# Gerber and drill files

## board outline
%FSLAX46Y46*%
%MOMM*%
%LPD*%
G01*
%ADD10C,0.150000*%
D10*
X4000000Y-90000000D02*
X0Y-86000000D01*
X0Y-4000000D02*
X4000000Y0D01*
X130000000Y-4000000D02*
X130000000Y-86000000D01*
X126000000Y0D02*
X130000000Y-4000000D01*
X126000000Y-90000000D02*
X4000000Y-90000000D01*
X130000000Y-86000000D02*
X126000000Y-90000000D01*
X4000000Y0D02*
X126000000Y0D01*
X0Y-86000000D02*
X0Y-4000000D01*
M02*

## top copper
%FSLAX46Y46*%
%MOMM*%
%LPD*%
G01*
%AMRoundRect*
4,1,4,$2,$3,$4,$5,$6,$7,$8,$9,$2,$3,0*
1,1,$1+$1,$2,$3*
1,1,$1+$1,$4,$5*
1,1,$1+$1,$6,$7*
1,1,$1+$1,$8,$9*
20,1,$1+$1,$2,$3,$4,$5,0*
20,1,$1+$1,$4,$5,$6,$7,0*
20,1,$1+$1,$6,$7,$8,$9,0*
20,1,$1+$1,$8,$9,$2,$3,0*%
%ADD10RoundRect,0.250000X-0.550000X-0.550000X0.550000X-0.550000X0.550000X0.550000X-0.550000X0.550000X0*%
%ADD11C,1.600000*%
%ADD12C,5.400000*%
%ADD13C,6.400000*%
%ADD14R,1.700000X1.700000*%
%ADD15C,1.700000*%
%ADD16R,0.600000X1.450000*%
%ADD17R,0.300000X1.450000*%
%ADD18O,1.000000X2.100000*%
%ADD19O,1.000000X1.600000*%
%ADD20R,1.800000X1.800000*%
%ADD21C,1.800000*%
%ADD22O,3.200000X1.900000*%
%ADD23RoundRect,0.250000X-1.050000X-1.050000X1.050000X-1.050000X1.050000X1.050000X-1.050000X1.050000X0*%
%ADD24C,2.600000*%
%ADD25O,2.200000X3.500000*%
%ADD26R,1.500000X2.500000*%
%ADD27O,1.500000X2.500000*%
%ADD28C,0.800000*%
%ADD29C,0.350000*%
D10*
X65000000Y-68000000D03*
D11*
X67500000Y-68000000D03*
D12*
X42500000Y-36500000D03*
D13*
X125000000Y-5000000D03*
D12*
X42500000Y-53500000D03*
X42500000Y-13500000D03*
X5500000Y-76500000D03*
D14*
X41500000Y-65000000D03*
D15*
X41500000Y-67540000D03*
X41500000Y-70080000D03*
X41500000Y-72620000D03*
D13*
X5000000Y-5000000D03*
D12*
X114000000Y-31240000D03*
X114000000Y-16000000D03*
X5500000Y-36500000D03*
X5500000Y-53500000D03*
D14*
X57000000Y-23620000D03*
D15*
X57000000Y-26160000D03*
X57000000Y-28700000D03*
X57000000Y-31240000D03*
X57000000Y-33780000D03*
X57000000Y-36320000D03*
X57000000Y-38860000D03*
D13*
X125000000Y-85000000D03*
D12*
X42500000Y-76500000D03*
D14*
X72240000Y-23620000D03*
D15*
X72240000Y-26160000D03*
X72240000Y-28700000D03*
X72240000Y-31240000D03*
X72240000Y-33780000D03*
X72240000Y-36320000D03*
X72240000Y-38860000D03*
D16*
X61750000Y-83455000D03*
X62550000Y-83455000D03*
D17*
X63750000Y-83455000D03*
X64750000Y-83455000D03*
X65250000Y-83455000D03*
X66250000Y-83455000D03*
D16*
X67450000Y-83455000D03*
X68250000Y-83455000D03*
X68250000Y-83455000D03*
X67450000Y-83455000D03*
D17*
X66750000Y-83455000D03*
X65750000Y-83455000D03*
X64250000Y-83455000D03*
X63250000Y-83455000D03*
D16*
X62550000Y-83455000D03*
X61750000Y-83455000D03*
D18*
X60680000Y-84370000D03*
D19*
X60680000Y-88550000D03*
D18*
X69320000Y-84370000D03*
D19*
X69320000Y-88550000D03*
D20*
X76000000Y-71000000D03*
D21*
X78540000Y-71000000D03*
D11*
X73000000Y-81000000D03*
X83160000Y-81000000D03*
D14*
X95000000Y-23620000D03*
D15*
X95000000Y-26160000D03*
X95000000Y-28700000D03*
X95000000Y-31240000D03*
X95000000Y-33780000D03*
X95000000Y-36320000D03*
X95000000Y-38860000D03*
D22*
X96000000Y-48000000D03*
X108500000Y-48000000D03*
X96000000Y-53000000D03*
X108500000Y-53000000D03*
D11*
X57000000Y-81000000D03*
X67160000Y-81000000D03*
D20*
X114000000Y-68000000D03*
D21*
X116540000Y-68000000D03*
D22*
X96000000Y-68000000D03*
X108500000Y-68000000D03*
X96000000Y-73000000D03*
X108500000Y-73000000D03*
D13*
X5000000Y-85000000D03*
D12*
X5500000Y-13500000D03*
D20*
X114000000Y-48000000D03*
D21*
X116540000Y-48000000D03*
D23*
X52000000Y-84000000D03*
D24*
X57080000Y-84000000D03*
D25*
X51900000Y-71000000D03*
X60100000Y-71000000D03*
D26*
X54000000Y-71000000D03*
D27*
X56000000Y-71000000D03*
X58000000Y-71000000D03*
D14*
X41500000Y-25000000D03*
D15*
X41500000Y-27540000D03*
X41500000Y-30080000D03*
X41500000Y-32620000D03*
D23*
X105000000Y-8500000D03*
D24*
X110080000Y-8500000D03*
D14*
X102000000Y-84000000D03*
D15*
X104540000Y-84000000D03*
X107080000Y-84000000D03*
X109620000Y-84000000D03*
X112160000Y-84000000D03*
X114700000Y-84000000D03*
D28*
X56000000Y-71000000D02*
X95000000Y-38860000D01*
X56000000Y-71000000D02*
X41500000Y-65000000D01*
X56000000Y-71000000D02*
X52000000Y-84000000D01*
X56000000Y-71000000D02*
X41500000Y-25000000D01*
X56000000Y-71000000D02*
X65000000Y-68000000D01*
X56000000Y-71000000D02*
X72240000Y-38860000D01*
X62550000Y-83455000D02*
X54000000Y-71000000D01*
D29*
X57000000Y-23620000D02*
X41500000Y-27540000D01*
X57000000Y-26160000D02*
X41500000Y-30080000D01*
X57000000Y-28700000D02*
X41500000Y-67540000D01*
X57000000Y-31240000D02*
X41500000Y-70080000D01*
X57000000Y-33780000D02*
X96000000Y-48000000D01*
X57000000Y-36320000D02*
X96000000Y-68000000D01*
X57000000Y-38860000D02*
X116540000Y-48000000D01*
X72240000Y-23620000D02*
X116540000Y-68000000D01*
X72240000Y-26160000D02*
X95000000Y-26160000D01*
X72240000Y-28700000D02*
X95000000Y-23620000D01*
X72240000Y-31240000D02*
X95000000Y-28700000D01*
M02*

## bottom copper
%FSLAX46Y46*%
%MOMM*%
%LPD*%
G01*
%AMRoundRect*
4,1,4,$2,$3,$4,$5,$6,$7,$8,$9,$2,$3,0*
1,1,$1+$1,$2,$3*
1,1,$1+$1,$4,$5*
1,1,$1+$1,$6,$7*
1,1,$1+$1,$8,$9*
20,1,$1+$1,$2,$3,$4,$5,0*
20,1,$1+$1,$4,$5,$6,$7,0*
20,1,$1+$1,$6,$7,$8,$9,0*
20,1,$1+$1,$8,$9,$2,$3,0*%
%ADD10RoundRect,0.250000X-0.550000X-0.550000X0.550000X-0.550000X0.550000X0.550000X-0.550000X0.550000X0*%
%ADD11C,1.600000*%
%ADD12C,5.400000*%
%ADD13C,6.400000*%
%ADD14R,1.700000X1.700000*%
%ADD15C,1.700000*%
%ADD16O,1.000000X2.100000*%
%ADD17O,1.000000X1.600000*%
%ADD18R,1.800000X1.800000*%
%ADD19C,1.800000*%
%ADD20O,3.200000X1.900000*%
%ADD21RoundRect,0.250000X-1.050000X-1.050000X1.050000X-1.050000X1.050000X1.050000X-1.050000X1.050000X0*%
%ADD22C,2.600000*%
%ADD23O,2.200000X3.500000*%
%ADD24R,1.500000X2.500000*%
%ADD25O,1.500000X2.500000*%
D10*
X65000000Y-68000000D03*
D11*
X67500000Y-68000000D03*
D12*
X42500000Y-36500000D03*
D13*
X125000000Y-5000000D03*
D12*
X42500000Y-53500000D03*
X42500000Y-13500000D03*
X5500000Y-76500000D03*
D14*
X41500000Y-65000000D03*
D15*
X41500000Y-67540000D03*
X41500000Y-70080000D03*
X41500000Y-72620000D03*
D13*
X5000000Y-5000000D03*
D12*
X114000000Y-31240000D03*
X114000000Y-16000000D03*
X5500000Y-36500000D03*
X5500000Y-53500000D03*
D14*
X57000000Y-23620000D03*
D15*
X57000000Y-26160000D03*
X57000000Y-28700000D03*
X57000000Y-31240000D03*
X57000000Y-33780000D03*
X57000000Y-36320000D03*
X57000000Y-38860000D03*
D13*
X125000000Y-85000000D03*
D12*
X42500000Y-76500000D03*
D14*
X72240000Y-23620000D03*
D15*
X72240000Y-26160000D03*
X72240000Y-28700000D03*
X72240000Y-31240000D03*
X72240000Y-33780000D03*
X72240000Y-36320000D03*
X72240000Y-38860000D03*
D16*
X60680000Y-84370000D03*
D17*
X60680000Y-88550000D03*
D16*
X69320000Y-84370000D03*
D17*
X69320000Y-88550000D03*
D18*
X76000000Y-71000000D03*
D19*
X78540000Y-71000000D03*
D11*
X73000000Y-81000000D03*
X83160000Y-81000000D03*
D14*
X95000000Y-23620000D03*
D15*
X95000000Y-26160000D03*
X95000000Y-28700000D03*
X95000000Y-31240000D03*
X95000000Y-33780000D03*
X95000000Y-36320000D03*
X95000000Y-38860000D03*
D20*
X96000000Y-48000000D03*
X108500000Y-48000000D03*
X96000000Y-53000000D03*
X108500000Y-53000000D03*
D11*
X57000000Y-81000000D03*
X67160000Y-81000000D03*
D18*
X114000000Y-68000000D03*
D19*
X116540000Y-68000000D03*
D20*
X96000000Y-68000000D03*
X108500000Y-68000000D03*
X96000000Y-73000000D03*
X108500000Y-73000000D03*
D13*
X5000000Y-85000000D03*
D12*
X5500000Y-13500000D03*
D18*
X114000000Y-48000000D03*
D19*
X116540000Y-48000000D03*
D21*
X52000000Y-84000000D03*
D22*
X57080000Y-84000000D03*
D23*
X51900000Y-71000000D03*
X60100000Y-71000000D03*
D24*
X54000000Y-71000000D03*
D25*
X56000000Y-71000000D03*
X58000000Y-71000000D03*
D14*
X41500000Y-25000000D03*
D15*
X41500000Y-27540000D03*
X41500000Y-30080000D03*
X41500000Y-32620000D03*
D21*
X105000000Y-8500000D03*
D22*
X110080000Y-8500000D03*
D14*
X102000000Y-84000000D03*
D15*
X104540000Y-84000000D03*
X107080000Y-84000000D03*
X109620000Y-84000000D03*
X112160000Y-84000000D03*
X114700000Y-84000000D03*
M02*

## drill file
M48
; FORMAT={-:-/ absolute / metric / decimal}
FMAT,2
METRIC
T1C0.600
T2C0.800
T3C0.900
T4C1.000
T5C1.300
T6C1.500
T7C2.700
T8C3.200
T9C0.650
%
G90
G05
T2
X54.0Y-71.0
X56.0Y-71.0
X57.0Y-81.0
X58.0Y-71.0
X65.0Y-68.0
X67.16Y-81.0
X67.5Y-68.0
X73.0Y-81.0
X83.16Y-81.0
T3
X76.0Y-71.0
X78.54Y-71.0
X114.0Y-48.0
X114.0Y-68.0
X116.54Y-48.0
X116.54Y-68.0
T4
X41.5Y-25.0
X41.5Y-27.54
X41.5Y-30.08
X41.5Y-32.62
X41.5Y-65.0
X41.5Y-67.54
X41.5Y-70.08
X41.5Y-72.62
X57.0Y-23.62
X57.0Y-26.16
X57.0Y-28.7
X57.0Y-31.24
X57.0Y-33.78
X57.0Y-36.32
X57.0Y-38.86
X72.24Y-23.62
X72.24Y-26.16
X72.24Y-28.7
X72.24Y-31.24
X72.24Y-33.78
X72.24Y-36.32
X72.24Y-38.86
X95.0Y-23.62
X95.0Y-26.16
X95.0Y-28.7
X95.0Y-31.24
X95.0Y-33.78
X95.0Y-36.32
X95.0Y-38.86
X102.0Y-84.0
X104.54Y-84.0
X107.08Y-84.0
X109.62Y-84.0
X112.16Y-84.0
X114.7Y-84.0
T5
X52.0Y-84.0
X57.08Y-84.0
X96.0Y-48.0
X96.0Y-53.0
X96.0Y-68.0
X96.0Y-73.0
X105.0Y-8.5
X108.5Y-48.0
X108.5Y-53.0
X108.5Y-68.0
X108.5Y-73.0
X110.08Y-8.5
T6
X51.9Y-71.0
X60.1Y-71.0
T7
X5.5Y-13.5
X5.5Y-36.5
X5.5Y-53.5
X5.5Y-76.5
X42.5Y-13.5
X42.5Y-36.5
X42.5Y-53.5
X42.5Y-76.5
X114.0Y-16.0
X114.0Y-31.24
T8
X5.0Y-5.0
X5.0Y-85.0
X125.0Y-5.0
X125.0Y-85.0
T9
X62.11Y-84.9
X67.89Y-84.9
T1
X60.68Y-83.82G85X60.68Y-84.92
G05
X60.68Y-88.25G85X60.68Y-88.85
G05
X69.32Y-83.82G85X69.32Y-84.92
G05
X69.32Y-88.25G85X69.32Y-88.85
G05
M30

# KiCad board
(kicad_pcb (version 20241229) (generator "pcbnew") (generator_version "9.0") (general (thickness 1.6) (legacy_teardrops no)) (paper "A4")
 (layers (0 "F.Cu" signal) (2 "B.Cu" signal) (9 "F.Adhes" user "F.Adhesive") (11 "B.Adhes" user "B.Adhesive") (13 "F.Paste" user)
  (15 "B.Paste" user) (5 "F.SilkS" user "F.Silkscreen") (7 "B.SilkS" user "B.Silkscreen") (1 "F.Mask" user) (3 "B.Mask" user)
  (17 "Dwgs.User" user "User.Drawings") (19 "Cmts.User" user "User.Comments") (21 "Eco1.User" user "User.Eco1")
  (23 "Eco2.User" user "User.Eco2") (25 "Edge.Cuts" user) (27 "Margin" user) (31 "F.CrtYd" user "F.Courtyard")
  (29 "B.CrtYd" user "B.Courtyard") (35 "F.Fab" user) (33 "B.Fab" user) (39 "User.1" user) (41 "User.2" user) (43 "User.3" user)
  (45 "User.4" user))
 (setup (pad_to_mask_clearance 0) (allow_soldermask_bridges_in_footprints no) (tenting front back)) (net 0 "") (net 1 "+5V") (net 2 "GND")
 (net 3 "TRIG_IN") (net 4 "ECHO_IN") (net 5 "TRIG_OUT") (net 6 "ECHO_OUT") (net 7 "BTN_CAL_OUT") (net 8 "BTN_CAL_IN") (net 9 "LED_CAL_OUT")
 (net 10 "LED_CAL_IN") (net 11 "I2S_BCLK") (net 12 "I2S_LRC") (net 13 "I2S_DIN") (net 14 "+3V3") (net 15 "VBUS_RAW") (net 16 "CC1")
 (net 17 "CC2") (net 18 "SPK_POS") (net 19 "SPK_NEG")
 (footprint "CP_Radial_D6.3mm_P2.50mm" (layer "F.Cu") (at 65 68)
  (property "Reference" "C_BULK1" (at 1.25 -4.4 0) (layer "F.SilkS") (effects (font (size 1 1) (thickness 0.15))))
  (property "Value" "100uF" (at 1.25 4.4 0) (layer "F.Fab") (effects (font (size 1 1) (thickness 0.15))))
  (pad "1" thru_hole roundrect (at 0 0) (size 1.6 1.6) (drill 0.8) (layers "*.Cu" "*.Mask") (remove_unused_layers no)
   (roundrect_rratio 0.15625) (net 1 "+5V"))
  (pad "2" thru_hole circle (at 2.5 0) (size 1.6 1.6) (drill 0.8) (layers "*.Cu" "*.Mask") (remove_unused_layers no) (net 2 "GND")))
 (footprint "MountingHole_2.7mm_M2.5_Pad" (layer "F.Cu") (at 42.5 36.5)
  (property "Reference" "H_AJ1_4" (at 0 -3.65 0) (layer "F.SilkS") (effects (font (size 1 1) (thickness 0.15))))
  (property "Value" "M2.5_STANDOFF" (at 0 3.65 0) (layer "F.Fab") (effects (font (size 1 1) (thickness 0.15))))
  (pad "1" thru_hole circle (at 0 0) (size 5.4 5.4) (drill 2.7) (layers "*.Cu" "*.Mask") (remove_unused_layers no) (zone_connect 2)))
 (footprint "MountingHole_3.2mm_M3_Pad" (layer "F.Cu") (at 125 5)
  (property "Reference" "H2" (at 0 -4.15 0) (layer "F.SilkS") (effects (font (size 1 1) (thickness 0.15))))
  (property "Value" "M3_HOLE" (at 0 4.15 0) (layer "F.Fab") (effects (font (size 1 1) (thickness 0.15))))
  (pad "1" thru_hole circle (at 0 0) (size 6.4 6.4) (drill 3.2) (layers "*.Cu" "*.Mask") (remove_unused_layers no) (zone_connect 2)))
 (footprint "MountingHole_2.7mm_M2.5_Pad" (layer "F.Cu") (at 42.5 53.5)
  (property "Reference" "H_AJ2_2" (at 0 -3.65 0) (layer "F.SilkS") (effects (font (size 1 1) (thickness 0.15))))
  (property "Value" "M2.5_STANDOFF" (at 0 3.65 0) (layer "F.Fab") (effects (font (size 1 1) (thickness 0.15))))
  (pad "1" thru_hole circle (at 0 0) (size 5.4 5.4) (drill 2.7) (layers "*.Cu" "*.Mask") (remove_unused_layers no) (zone_connect 2)))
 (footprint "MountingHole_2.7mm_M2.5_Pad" (layer "F.Cu") (at 42.5 13.5)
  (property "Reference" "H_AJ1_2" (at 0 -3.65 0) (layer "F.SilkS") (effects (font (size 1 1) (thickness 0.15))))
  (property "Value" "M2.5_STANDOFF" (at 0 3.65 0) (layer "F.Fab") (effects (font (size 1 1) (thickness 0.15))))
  (pad "1" thru_hole circle (at 0 0) (size 5.4 5.4) (drill 2.7) (layers "*.Cu" "*.Mask") (remove_unused_layers no) (zone_connect 2)))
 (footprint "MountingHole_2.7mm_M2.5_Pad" (layer "F.Cu") (at 5.5 76.5)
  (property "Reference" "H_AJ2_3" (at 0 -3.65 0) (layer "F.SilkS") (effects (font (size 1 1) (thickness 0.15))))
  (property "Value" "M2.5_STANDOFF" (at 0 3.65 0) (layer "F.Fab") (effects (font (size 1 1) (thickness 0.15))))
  (pad "1" thru_hole circle (at 0 0) (size 5.4 5.4) (drill 2.7) (layers "*.Cu" "*.Mask") (remove_unused_layers no) (zone_connect 2)))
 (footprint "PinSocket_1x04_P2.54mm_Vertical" (layer "F.Cu") (at 41.5 65)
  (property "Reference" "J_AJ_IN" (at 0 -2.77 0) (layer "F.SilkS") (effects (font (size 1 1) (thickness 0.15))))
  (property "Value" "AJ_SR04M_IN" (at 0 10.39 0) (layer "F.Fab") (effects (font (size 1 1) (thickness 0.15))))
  (pad "1" thru_hole rect (at 0 0) (size 1.7 1.7) (drill 1) (layers "*.Cu" "*.Mask") (remove_unused_layers no) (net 1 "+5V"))
  (pad "2" thru_hole circle (at 0 2.54) (size 1.7 1.7) (drill 1) (layers "*.Cu" "*.Mask") (remove_unused_layers no) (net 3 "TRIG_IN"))
  (pad "3" thru_hole circle (at 0 5.08) (size 1.7 1.7) (drill 1) (layers "*.Cu" "*.Mask") (remove_unused_layers no) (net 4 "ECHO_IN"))
  (pad "4" thru_hole circle (at 0 7.62) (size 1.7 1.7) (drill 1) (layers "*.Cu" "*.Mask") (remove_unused_layers no) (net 2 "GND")))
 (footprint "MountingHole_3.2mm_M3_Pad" (layer "F.Cu") (at 5 5)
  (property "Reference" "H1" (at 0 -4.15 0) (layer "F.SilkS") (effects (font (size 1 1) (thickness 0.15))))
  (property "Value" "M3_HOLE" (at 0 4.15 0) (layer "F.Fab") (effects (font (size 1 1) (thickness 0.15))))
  (pad "1" thru_hole circle (at 0 0) (size 6.4 6.4) (drill 3.2) (layers "*.Cu" "*.Mask") (remove_unused_layers no) (zone_connect 2)))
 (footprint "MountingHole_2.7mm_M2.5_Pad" (layer "F.Cu") (at 114 31.24)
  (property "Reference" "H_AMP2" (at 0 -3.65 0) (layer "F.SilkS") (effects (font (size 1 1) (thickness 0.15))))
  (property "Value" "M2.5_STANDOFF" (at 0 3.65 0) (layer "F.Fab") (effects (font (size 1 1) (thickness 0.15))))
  (pad "1" thru_hole circle (at 0 0) (size 5.4 5.4) (drill 2.7) (layers "*.Cu" "*.Mask") (remove_unused_layers no) (zone_connect 2)))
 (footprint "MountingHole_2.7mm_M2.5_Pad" (layer "F.Cu") (at 114 16)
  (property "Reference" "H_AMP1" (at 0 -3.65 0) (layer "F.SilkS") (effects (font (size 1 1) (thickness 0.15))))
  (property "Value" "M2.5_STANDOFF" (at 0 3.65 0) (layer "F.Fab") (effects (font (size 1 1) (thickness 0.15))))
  (pad "1" thru_hole circle (at 0 0) (size 5.4 5.4) (drill 2.7) (layers "*.Cu" "*.Mask") (remove_unused_layers no) (zone_connect 2)))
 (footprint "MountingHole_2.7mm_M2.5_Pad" (layer "F.Cu") (at 5.5 36.5)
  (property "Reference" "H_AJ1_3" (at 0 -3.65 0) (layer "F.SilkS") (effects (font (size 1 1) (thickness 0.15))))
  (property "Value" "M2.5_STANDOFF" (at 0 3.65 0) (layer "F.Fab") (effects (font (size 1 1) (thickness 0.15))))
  (pad "1" thru_hole circle (at 0 0) (size 5.4 5.4) (drill 2.7) (layers "*.Cu" "*.Mask") (remove_unused_layers no) (zone_connect 2)))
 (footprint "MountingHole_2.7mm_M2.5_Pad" (layer "F.Cu") (at 5.5 53.5)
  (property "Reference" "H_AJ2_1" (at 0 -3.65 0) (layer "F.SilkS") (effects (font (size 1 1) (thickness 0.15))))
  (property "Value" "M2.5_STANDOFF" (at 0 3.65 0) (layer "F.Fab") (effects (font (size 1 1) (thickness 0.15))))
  (pad "1" thru_hole circle (at 0 0) (size 5.4 5.4) (drill 2.7) (layers "*.Cu" "*.Mask") (remove_unused_layers no) (zone_connect 2)))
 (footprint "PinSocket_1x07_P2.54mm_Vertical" (layer "F.Cu") (at 57 23.62)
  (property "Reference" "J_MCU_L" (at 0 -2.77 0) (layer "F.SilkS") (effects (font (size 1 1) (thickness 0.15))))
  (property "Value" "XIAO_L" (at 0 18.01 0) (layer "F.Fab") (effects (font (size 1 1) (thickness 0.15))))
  (pad "1" thru_hole rect (at 0 0) (size 1.7 1.7) (drill 1) (layers "*.Cu" "*.Mask") (remove_unused_layers no) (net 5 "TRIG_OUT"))
  (pad "2" thru_hole circle (at 0 2.54) (size 1.7 1.7) (drill 1) (layers "*.Cu" "*.Mask") (remove_unused_layers no) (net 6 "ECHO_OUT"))
  (pad "3" thru_hole circle (at 0 5.08) (size 1.7 1.7) (drill 1) (layers "*.Cu" "*.Mask") (remove_unused_layers no) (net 3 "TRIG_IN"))
  (pad "4" thru_hole circle (at 0 7.62) (size 1.7 1.7) (drill 1) (layers "*.Cu" "*.Mask") (remove_unused_layers no) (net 4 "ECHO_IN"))
  (pad "5" thru_hole circle (at 0 10.16) (size 1.7 1.7) (drill 1) (layers "*.Cu" "*.Mask") (remove_unused_layers no) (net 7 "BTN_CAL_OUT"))
  (pad "6" thru_hole circle (at 0 12.7) (size 1.7 1.7) (drill 1) (layers "*.Cu" "*.Mask") (remove_unused_layers no) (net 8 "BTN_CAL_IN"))
  (pad "7" thru_hole circle (at 0 15.24) (size 1.7 1.7) (drill 1) (layers "*.Cu" "*.Mask") (remove_unused_layers no) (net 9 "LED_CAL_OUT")))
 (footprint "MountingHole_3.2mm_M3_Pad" (layer "F.Cu") (at 125 85)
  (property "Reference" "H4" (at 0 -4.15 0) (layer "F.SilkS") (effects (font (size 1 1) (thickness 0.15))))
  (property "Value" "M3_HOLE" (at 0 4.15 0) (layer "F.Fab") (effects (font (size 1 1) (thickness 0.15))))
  (pad "1" thru_hole circle (at 0 0) (size 6.4 6.4) (drill 3.2) (layers "*.Cu" "*.Mask") (remove_unused_layers no) (zone_connect 2)))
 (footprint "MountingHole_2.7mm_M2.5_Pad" (layer "F.Cu") (at 42.5 76.5)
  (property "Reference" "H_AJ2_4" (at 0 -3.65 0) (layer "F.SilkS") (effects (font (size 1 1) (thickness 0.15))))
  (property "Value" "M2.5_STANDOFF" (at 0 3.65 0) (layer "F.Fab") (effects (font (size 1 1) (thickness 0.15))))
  (pad "1" thru_hole circle (at 0 0) (size 5.4 5.4) (drill 2.7) (layers "*.Cu" "*.Mask") (remove_unused_layers no) (zone_connect 2)))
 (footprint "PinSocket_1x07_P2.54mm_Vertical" (layer "F.Cu") (at 72.24 23.62)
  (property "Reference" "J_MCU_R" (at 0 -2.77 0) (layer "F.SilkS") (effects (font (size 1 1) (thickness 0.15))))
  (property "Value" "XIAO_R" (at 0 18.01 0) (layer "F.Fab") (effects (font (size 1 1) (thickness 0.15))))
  (pad "1" thru_hole rect (at 0 0) (size 1.7 1.7) (drill 1) (layers "*.Cu" "*.Mask") (remove_unused_layers no) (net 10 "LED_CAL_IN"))
  (pad "2" thru_hole circle (at 0 2.54) (size 1.7 1.7) (drill 1) (layers "*.Cu" "*.Mask") (remove_unused_layers no) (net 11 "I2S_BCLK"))
  (pad "3" thru_hole circle (at 0 5.08) (size 1.7 1.7) (drill 1) (layers "*.Cu" "*.Mask") (remove_unused_layers no) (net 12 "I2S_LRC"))
  (pad "4" thru_hole circle (at 0 7.62) (size 1.7 1.7) (drill 1) (layers "*.Cu" "*.Mask") (remove_unused_layers no) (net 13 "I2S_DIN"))
  (pad "5" thru_hole circle (at 0 10.16) (size 1.7 1.7) (drill 1) (layers "*.Cu" "*.Mask") (remove_unused_layers no) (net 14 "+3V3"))
  (pad "6" thru_hole circle (at 0 12.7) (size 1.7 1.7) (drill 1) (layers "*.Cu" "*.Mask") (remove_unused_layers no) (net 2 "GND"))
  (pad "7" thru_hole circle (at 0 15.24) (size 1.7 1.7) (drill 1) (layers "*.Cu" "*.Mask") (remove_unused_layers no) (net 1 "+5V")))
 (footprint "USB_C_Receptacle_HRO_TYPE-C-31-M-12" (layer "F.Cu") (at 65 87.5)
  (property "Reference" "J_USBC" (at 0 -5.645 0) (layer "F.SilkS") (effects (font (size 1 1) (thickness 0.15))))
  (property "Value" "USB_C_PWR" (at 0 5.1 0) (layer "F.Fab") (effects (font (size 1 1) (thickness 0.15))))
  (pad "" np_thru_hole circle (at -2.89 -2.6) (size 0.65 0.65) (drill 0.65) (layers "*.Cu" "*.Mask"))
  (pad "" np_thru_hole circle (at 2.89 -2.6) (size 0.65 0.65) (drill 0.65) (layers "*.Cu" "*.Mask"))
  (pad "A1" smd rect (at -3.25 -4.045) (size 0.6 1.45) (layers "F.Cu" "F.Mask" "F.Paste") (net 2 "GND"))
  (pad "A4" smd rect (at -2.45 -4.045) (size 0.6 1.45) (layers "F.Cu" "F.Mask" "F.Paste") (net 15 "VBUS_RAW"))
  (pad "A5" smd rect (at -1.25 -4.045) (size 0.3 1.45) (layers "F.Cu" "F.Mask" "F.Paste") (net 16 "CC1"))
  (pad "A6" smd rect (at -0.25 -4.045) (size 0.3 1.45) (layers "F.Cu" "F.Mask" "F.Paste"))
  (pad "A7" smd rect (at 0.25 -4.045) (size 0.3 1.45) (layers "F.Cu" "F.Mask" "F.Paste"))
  (pad "A8" smd rect (at 1.25 -4.045) (size 0.3 1.45) (layers "F.Cu" "F.Mask" "F.Paste"))
  (pad "A9" smd rect (at 2.45 -4.045) (size 0.6 1.45) (layers "F.Cu" "F.Mask" "F.Paste") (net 15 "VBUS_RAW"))
  (pad "A12" smd rect (at 3.25 -4.045) (size 0.6 1.45) (layers "F.Cu" "F.Mask" "F.Paste") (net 2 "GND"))
  (pad "B1" smd rect (at 3.25 -4.045) (size 0.6 1.45) (layers "F.Cu" "F.Mask" "F.Paste") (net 2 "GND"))
  (pad "B4" smd rect (at 2.45 -4.045) (size 0.6 1.45) (layers "F.Cu" "F.Mask" "F.Paste") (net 15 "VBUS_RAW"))
  (pad "B5" smd rect (at 1.75 -4.045) (size 0.3 1.45) (layers "F.Cu" "F.Mask" "F.Paste") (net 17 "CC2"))
  (pad "B6" smd rect (at 0.75 -4.045) (size 0.3 1.45) (layers "F.Cu" "F.Mask" "F.Paste"))
  (pad "B7" smd rect (at -0.75 -4.045) (size 0.3 1.45) (layers "F.Cu" "F.Mask" "F.Paste"))
  (pad "B8" smd rect (at -1.75 -4.045) (size 0.3 1.45) (layers "F.Cu" "F.Mask" "F.Paste"))
  (pad "B9" smd rect (at -2.45 -4.045) (size 0.6 1.45) (layers "F.Cu" "F.Mask" "F.Paste") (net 15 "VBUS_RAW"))
  (pad "B12" smd rect (at -3.25 -4.045) (size 0.6 1.45) (layers "F.Cu" "F.Mask" "F.Paste") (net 2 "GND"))
  (pad "S1" thru_hole oval (at -4.32 -3.13) (size 1 2.1) (drill oval 0.6 1.7) (layers "*.Cu" "*.Mask") (remove_unused_layers no)
   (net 2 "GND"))
  (pad "S1" thru_hole oval (at -4.32 1.05) (size 1 1.6) (drill oval 0.6 1.2) (layers "*.Cu" "*.Mask") (remove_unused_layers no)
   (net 2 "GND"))
  (pad "S1" thru_hole oval (at 4.32 -3.13) (size 1 2.1) (drill oval 0.6 1.7) (layers "*.Cu" "*.Mask") (remove_unused_layers no)
   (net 2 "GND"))
  (pad "S1" thru_hole oval (at 4.32 1.05) (size 1 1.6) (drill oval 0.6 1.2) (layers "*.Cu" "*.Mask") (remove_unused_layers no) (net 2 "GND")))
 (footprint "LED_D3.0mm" (layer "F.Cu") (at 76 71)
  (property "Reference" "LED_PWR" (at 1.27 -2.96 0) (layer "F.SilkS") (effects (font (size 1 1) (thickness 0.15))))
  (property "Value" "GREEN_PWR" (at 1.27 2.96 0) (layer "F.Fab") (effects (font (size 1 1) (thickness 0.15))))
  (pad "1" thru_hole rect (at 0 0) (size 1.8 1.8) (drill 0.9) (layers "*.Cu" "*.Mask") (remove_unused_layers no) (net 2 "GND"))
  (pad "2" thru_hole circle (at 2.54 0) (size 1.8 1.8) (drill 0.9) (layers "*.Cu" "*.Mask") (remove_unused_layers no) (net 1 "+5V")))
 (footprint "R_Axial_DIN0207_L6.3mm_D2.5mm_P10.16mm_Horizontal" (layer "F.Cu") (at 73 81)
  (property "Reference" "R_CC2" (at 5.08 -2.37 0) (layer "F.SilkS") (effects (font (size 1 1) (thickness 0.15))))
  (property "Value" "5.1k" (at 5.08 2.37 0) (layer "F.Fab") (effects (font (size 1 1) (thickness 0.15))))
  (pad "1" thru_hole circle (at 0 0) (size 1.6 1.6) (drill 0.8) (layers "*.Cu" "*.Mask") (remove_unused_layers no) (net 17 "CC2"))
  (pad "2" thru_hole circle (at 10.16 0) (size 1.6 1.6) (drill 0.8) (layers "*.Cu" "*.Mask") (remove_unused_layers no) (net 2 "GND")))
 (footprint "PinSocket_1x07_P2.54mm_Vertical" (layer "F.Cu") (at 95 23.62)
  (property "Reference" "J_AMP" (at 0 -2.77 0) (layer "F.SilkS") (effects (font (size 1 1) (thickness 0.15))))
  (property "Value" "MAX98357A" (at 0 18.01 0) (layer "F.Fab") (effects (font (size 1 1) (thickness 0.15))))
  (pad "1" thru_hole rect (at 0 0) (size 1.7 1.7) (drill 1) (layers "*.Cu" "*.Mask") (remove_unused_layers no) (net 12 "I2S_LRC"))
  (pad "2" thru_hole circle (at 0 2.54) (size 1.7 1.7) (drill 1) (layers "*.Cu" "*.Mask") (remove_unused_layers no) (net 11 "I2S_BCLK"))
  (pad "3" thru_hole circle (at 0 5.08) (size 1.7 1.7) (drill 1) (layers "*.Cu" "*.Mask") (remove_unused_layers no) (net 13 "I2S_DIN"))
  (pad "4" thru_hole circle (at 0 7.62) (size 1.7 1.7) (drill 1) (layers "*.Cu" "*.Mask") (remove_unused_layers no) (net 2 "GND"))
  (pad "5" thru_hole circle (at 0 10.16) (size 1.7 1.7) (drill 1) (layers "*.Cu" "*.Mask") (remove_unused_layers no) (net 2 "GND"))
  (pad "6" thru_hole circle (at 0 12.7) (size 1.7 1.7) (drill 1) (layers "*.Cu" "*.Mask") (remove_unused_layers no) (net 2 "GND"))
  (pad "7" thru_hole circle (at 0 15.24) (size 1.7 1.7) (drill 1) (layers "*.Cu" "*.Mask") (remove_unused_layers no) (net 1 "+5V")))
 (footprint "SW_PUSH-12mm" (layer "F.Cu") (at 96 48)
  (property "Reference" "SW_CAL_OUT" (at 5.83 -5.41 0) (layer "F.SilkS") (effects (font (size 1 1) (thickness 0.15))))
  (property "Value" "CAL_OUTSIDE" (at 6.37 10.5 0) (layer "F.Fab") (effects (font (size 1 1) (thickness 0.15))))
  (pad "1" thru_hole oval (at 0 0) (size 3.2 1.9) (drill 1.3) (layers "*.Cu" "*.Mask") (remove_unused_layers no) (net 7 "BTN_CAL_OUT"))
  (pad "1" thru_hole oval (at 12.5 0) (size 3.2 1.9) (drill 1.3) (layers "*.Cu" "*.Mask") (remove_unused_layers no) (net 7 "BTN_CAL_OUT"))
  (pad "2" thru_hole oval (at 0 5) (size 3.2 1.9) (drill 1.3) (layers "*.Cu" "*.Mask") (remove_unused_layers no) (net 2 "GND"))
  (pad "2" thru_hole oval (at 12.5 5) (size 3.2 1.9) (drill 1.3) (layers "*.Cu" "*.Mask") (remove_unused_layers no) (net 2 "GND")))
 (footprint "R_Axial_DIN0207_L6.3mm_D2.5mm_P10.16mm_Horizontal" (layer "F.Cu") (at 57 81)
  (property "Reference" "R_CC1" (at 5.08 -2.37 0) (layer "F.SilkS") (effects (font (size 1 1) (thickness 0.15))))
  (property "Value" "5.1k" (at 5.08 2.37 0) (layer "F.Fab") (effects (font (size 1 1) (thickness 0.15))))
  (pad "1" thru_hole circle (at 0 0) (size 1.6 1.6) (drill 0.8) (layers "*.Cu" "*.Mask") (remove_unused_layers no) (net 16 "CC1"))
  (pad "2" thru_hole circle (at 10.16 0) (size 1.6 1.6) (drill 0.8) (layers "*.Cu" "*.Mask") (remove_unused_layers no) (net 2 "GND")))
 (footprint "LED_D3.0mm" (layer "F.Cu") (at 114 68)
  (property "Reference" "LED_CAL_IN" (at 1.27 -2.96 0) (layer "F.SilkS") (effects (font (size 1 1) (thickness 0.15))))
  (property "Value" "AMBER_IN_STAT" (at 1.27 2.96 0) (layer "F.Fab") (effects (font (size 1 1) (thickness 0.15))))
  (pad "1" thru_hole rect (at 0 0) (size 1.8 1.8) (drill 0.9) (layers "*.Cu" "*.Mask") (remove_unused_layers no) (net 2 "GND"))
  (pad "2" thru_hole circle (at 2.54 0) (size 1.8 1.8) (drill 0.9) (layers "*.Cu" "*.Mask") (remove_unused_layers no) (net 10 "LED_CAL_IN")))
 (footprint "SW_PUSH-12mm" (layer "F.Cu") (at 96 68)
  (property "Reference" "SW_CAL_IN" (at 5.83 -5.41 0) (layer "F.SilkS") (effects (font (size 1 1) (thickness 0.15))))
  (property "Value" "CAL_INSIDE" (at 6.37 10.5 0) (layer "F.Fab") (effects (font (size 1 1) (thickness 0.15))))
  (pad "1" thru_hole oval (at 0 0) (size 3.2 1.9) (drill 1.3) (layers "*.Cu" "*.Mask") (remove_unused_layers no) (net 8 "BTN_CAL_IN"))
  (pad "1" thru_hole oval (at 12.5 0) (size 3.2 1.9) (drill 1.3) (layers "*.Cu" "*.Mask") (remove_unused_layers no) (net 8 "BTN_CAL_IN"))
  (pad "2" thru_hole oval (at 0 5) (size 3.2 1.9) (drill 1.3) (layers "*.Cu" "*.Mask") (remove_unused_layers no) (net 2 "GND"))
  (pad "2" thru_hole oval (at 12.5 5) (size 3.2 1.9) (drill 1.3) (layers "*.Cu" "*.Mask") (remove_unused_layers no) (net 2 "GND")))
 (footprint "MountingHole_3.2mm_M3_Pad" (layer "F.Cu") (at 5 85)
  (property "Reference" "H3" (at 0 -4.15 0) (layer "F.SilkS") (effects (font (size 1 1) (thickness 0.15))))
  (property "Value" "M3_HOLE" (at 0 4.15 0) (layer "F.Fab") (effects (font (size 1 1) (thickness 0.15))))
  (pad "1" thru_hole circle (at 0 0) (size 6.4 6.4) (drill 3.2) (layers "*.Cu" "*.Mask") (remove_unused_layers no) (zone_connect 2)))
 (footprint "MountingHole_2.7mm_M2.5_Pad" (layer "F.Cu") (at 5.5 13.5)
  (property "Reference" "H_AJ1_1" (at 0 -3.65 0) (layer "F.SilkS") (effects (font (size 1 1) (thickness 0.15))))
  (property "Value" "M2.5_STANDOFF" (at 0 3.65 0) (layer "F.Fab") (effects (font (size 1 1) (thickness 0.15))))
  (pad "1" thru_hole circle (at 0 0) (size 5.4 5.4) (drill 2.7) (layers "*.Cu" "*.Mask") (remove_unused_layers no) (zone_connect 2)))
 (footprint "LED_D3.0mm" (layer "F.Cu") (at 114 48)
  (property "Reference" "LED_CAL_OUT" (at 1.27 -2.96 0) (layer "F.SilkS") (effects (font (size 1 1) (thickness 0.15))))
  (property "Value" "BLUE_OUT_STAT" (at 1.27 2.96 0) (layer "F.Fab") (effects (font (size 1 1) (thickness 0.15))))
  (pad "1" thru_hole rect (at 0 0) (size 1.8 1.8) (drill 0.9) (layers "*.Cu" "*.Mask") (remove_unused_layers no) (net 2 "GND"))
  (pad "2" thru_hole circle (at 2.54 0) (size 1.8 1.8) (drill 0.9) (layers "*.Cu" "*.Mask") (remove_unused_layers no) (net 9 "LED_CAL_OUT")))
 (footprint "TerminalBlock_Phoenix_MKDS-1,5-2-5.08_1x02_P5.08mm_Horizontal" (layer "F.Cu") (at 52 84)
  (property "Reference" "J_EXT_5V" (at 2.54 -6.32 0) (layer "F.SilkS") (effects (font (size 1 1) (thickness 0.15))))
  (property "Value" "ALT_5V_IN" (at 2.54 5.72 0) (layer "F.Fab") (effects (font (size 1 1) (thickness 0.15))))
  (pad "1" thru_hole roundrect (at 0 0) (size 2.6 2.6) (drill 1.3) (layers "*.Cu" "*.Mask") (remove_unused_layers no)
   (roundrect_rratio 0.096154) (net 1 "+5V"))
  (pad "2" thru_hole circle (at 5.08 0) (size 2.6 2.6) (drill 1.3) (layers "*.Cu" "*.Mask") (remove_unused_layers no) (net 2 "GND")))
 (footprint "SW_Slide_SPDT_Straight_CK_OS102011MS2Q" (layer "F.Cu") (at 54 71)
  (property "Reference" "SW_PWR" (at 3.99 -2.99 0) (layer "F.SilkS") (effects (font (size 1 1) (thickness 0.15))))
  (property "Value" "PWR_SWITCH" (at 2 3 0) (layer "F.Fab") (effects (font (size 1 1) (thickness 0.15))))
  (pad "" thru_hole oval (at -2.1 0) (size 2.2 3.5) (drill 1.5) (layers "*.Cu" "*.Mask") (remove_unused_layers no))
  (pad "" thru_hole oval (at 6.1 0) (size 2.2 3.5) (drill 1.5) (layers "*.Cu" "*.Mask") (remove_unused_layers no))
  (pad "1" thru_hole rect (at 0 0) (size 1.5 2.5) (drill 0.8) (layers "*.Cu" "*.Mask") (remove_unused_layers no) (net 15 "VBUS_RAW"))
  (pad "2" thru_hole oval (at 2 0) (size 1.5 2.5) (drill 0.8) (layers "*.Cu" "*.Mask") (remove_unused_layers no) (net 1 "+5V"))
  (pad "3" thru_hole oval (at 4 0) (size 1.5 2.5) (drill 0.8) (layers "*.Cu" "*.Mask") (remove_unused_layers no) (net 15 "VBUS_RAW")))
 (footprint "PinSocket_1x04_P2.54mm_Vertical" (layer "F.Cu") (at 41.5 25)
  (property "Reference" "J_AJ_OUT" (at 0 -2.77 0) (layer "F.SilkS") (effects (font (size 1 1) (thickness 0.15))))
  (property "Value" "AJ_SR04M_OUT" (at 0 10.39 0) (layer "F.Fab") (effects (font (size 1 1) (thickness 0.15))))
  (pad "1" thru_hole rect (at 0 0) (size 1.7 1.7) (drill 1) (layers "*.Cu" "*.Mask") (remove_unused_layers no) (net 1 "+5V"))
  (pad "2" thru_hole circle (at 0 2.54) (size 1.7 1.7) (drill 1) (layers "*.Cu" "*.Mask") (remove_unused_layers no) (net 5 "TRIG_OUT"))
  (pad "3" thru_hole circle (at 0 5.08) (size 1.7 1.7) (drill 1) (layers "*.Cu" "*.Mask") (remove_unused_layers no) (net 6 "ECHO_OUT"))
  (pad "4" thru_hole circle (at 0 7.62) (size 1.7 1.7) (drill 1) (layers "*.Cu" "*.Mask") (remove_unused_layers no) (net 2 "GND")))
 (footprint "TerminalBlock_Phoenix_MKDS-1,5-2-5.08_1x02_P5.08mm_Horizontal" (layer "F.Cu") (at 105 8.5)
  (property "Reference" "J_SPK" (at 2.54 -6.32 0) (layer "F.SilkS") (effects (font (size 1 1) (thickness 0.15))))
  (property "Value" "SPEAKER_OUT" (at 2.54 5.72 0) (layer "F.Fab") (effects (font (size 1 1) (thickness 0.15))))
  (pad "1" thru_hole roundrect (at 0 0) (size 2.6 2.6) (drill 1.3) (layers "*.Cu" "*.Mask") (remove_unused_layers no)
   (roundrect_rratio 0.096154) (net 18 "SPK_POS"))
  (pad "2" thru_hole circle (at 5.08 0) (size 2.6 2.6) (drill 1.3) (layers "*.Cu" "*.Mask") (remove_unused_layers no) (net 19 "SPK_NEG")))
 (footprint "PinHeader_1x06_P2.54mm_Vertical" (layer "F.Cu") (at 102 84 90)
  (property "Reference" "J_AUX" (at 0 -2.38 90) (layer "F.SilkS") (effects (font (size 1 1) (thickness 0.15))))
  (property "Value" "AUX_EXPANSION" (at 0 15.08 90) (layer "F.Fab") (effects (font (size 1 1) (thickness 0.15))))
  (pad "1" thru_hole rect (at 0 0 90) (size 1.7 1.7) (drill 1) (layers "*.Cu" "*.Mask") (remove_unused_layers no) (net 14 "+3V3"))
  (pad "2" thru_hole circle (at 0 2.54 90) (size 1.7 1.7) (drill 1) (layers "*.Cu" "*.Mask") (remove_unused_layers no) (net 9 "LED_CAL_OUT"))
  (pad "3" thru_hole circle (at 0 5.08 90) (size 1.7 1.7) (drill 1) (layers "*.Cu" "*.Mask") (remove_unused_layers no) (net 10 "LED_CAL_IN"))
  (pad "4" thru_hole circle (at 0 7.62 90) (size 1.7 1.7) (drill 1) (layers "*.Cu" "*.Mask") (remove_unused_layers no) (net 7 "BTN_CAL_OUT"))
  (pad "5" thru_hole circle (at 0 10.16 90) (size 1.7 1.7) (drill 1) (layers "*.Cu" "*.Mask") (remove_unused_layers no) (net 8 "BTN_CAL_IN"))
  (pad "6" thru_hole circle (at 0 12.7 90) (size 1.7 1.7) (drill 1) (layers "*.Cu" "*.Mask") (remove_unused_layers no) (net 2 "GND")))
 (gr_line (start 4 90) (end 0 86) (stroke (width 0.15) (type default)) (layer "Edge.Cuts"))
 (gr_line (start 0 4) (end 4 0) (stroke (width 0.15) (type default)) (layer "Edge.Cuts"))
 (gr_line (start 130 4) (end 130 86) (stroke (width 0.15) (type default)) (layer "Edge.Cuts"))
 (gr_line (start 126 0) (end 130 4) (stroke (width 0.15) (type default)) (layer "Edge.Cuts"))
 (gr_line (start 126 90) (end 4 90) (stroke (width 0.15) (type default)) (layer "Edge.Cuts"))
 (gr_line (start 130 86) (end 126 90) (stroke (width 0.15) (type default)) (layer "Edge.Cuts"))
 (gr_line (start 4 0) (end 126 0) (stroke (width 0.15) (type default)) (layer "Edge.Cuts"))
 (gr_line (start 0 86) (end 0 4) (stroke (width 0.15) (type default)) (layer "Edge.Cuts"))
 (segment (start 56 71) (end 95 38.86) (width 0.8) (layer "F.Cu") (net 1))
 (segment (start 56 71) (end 41.5 65) (width 0.8) (layer "F.Cu") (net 1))
 (segment (start 56 71) (end 52 84) (width 0.8) (layer "F.Cu") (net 1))
 (segment (start 56 71) (end 41.5 25) (width 0.8) (layer "F.Cu") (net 1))
 (segment (start 56 71) (end 65 68) (width 0.8) (layer "F.Cu") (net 1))
 (segment (start 56 71) (end 72.24 38.86) (width 0.8) (layer "F.Cu") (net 1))
 (segment (start 62.55 83.455) (end 54 71) (width 0.8) (layer "F.Cu") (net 15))
 (segment (start 57 23.62) (end 41.5 27.54) (width 0.35) (layer "F.Cu") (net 5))
 (segment (start 57 26.16) (end 41.5 30.08) (width 0.35) (layer "F.Cu") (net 6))
 (segment (start 57 28.7) (end 41.5 67.54) (width 0.35) (layer "F.Cu") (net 3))
 (segment (start 57 31.24) (end 41.5 70.08) (width 0.35) (layer "F.Cu") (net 4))
 (segment (start 57 33.78) (end 96 48) (width 0.35) (layer "F.Cu") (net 7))
 (segment (start 57 36.32) (end 96 68) (width 0.35) (layer "F.Cu") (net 8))
 (segment (start 57 38.86) (end 116.54 48) (width 0.35) (layer "F.Cu") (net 9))
 (segment (start 72.24 23.62) (end 116.54 68) (width 0.35) (layer "F.Cu") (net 10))
 (segment (start 72.24 26.16) (end 95 26.16) (width 0.35) (layer "F.Cu") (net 11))
 (segment (start 72.24 28.7) (end 95 23.62) (width 0.35) (layer "F.Cu") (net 12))
 (segment (start 72.24 31.24) (end 95 28.7) (width 0.35) (layer "F.Cu") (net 13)))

